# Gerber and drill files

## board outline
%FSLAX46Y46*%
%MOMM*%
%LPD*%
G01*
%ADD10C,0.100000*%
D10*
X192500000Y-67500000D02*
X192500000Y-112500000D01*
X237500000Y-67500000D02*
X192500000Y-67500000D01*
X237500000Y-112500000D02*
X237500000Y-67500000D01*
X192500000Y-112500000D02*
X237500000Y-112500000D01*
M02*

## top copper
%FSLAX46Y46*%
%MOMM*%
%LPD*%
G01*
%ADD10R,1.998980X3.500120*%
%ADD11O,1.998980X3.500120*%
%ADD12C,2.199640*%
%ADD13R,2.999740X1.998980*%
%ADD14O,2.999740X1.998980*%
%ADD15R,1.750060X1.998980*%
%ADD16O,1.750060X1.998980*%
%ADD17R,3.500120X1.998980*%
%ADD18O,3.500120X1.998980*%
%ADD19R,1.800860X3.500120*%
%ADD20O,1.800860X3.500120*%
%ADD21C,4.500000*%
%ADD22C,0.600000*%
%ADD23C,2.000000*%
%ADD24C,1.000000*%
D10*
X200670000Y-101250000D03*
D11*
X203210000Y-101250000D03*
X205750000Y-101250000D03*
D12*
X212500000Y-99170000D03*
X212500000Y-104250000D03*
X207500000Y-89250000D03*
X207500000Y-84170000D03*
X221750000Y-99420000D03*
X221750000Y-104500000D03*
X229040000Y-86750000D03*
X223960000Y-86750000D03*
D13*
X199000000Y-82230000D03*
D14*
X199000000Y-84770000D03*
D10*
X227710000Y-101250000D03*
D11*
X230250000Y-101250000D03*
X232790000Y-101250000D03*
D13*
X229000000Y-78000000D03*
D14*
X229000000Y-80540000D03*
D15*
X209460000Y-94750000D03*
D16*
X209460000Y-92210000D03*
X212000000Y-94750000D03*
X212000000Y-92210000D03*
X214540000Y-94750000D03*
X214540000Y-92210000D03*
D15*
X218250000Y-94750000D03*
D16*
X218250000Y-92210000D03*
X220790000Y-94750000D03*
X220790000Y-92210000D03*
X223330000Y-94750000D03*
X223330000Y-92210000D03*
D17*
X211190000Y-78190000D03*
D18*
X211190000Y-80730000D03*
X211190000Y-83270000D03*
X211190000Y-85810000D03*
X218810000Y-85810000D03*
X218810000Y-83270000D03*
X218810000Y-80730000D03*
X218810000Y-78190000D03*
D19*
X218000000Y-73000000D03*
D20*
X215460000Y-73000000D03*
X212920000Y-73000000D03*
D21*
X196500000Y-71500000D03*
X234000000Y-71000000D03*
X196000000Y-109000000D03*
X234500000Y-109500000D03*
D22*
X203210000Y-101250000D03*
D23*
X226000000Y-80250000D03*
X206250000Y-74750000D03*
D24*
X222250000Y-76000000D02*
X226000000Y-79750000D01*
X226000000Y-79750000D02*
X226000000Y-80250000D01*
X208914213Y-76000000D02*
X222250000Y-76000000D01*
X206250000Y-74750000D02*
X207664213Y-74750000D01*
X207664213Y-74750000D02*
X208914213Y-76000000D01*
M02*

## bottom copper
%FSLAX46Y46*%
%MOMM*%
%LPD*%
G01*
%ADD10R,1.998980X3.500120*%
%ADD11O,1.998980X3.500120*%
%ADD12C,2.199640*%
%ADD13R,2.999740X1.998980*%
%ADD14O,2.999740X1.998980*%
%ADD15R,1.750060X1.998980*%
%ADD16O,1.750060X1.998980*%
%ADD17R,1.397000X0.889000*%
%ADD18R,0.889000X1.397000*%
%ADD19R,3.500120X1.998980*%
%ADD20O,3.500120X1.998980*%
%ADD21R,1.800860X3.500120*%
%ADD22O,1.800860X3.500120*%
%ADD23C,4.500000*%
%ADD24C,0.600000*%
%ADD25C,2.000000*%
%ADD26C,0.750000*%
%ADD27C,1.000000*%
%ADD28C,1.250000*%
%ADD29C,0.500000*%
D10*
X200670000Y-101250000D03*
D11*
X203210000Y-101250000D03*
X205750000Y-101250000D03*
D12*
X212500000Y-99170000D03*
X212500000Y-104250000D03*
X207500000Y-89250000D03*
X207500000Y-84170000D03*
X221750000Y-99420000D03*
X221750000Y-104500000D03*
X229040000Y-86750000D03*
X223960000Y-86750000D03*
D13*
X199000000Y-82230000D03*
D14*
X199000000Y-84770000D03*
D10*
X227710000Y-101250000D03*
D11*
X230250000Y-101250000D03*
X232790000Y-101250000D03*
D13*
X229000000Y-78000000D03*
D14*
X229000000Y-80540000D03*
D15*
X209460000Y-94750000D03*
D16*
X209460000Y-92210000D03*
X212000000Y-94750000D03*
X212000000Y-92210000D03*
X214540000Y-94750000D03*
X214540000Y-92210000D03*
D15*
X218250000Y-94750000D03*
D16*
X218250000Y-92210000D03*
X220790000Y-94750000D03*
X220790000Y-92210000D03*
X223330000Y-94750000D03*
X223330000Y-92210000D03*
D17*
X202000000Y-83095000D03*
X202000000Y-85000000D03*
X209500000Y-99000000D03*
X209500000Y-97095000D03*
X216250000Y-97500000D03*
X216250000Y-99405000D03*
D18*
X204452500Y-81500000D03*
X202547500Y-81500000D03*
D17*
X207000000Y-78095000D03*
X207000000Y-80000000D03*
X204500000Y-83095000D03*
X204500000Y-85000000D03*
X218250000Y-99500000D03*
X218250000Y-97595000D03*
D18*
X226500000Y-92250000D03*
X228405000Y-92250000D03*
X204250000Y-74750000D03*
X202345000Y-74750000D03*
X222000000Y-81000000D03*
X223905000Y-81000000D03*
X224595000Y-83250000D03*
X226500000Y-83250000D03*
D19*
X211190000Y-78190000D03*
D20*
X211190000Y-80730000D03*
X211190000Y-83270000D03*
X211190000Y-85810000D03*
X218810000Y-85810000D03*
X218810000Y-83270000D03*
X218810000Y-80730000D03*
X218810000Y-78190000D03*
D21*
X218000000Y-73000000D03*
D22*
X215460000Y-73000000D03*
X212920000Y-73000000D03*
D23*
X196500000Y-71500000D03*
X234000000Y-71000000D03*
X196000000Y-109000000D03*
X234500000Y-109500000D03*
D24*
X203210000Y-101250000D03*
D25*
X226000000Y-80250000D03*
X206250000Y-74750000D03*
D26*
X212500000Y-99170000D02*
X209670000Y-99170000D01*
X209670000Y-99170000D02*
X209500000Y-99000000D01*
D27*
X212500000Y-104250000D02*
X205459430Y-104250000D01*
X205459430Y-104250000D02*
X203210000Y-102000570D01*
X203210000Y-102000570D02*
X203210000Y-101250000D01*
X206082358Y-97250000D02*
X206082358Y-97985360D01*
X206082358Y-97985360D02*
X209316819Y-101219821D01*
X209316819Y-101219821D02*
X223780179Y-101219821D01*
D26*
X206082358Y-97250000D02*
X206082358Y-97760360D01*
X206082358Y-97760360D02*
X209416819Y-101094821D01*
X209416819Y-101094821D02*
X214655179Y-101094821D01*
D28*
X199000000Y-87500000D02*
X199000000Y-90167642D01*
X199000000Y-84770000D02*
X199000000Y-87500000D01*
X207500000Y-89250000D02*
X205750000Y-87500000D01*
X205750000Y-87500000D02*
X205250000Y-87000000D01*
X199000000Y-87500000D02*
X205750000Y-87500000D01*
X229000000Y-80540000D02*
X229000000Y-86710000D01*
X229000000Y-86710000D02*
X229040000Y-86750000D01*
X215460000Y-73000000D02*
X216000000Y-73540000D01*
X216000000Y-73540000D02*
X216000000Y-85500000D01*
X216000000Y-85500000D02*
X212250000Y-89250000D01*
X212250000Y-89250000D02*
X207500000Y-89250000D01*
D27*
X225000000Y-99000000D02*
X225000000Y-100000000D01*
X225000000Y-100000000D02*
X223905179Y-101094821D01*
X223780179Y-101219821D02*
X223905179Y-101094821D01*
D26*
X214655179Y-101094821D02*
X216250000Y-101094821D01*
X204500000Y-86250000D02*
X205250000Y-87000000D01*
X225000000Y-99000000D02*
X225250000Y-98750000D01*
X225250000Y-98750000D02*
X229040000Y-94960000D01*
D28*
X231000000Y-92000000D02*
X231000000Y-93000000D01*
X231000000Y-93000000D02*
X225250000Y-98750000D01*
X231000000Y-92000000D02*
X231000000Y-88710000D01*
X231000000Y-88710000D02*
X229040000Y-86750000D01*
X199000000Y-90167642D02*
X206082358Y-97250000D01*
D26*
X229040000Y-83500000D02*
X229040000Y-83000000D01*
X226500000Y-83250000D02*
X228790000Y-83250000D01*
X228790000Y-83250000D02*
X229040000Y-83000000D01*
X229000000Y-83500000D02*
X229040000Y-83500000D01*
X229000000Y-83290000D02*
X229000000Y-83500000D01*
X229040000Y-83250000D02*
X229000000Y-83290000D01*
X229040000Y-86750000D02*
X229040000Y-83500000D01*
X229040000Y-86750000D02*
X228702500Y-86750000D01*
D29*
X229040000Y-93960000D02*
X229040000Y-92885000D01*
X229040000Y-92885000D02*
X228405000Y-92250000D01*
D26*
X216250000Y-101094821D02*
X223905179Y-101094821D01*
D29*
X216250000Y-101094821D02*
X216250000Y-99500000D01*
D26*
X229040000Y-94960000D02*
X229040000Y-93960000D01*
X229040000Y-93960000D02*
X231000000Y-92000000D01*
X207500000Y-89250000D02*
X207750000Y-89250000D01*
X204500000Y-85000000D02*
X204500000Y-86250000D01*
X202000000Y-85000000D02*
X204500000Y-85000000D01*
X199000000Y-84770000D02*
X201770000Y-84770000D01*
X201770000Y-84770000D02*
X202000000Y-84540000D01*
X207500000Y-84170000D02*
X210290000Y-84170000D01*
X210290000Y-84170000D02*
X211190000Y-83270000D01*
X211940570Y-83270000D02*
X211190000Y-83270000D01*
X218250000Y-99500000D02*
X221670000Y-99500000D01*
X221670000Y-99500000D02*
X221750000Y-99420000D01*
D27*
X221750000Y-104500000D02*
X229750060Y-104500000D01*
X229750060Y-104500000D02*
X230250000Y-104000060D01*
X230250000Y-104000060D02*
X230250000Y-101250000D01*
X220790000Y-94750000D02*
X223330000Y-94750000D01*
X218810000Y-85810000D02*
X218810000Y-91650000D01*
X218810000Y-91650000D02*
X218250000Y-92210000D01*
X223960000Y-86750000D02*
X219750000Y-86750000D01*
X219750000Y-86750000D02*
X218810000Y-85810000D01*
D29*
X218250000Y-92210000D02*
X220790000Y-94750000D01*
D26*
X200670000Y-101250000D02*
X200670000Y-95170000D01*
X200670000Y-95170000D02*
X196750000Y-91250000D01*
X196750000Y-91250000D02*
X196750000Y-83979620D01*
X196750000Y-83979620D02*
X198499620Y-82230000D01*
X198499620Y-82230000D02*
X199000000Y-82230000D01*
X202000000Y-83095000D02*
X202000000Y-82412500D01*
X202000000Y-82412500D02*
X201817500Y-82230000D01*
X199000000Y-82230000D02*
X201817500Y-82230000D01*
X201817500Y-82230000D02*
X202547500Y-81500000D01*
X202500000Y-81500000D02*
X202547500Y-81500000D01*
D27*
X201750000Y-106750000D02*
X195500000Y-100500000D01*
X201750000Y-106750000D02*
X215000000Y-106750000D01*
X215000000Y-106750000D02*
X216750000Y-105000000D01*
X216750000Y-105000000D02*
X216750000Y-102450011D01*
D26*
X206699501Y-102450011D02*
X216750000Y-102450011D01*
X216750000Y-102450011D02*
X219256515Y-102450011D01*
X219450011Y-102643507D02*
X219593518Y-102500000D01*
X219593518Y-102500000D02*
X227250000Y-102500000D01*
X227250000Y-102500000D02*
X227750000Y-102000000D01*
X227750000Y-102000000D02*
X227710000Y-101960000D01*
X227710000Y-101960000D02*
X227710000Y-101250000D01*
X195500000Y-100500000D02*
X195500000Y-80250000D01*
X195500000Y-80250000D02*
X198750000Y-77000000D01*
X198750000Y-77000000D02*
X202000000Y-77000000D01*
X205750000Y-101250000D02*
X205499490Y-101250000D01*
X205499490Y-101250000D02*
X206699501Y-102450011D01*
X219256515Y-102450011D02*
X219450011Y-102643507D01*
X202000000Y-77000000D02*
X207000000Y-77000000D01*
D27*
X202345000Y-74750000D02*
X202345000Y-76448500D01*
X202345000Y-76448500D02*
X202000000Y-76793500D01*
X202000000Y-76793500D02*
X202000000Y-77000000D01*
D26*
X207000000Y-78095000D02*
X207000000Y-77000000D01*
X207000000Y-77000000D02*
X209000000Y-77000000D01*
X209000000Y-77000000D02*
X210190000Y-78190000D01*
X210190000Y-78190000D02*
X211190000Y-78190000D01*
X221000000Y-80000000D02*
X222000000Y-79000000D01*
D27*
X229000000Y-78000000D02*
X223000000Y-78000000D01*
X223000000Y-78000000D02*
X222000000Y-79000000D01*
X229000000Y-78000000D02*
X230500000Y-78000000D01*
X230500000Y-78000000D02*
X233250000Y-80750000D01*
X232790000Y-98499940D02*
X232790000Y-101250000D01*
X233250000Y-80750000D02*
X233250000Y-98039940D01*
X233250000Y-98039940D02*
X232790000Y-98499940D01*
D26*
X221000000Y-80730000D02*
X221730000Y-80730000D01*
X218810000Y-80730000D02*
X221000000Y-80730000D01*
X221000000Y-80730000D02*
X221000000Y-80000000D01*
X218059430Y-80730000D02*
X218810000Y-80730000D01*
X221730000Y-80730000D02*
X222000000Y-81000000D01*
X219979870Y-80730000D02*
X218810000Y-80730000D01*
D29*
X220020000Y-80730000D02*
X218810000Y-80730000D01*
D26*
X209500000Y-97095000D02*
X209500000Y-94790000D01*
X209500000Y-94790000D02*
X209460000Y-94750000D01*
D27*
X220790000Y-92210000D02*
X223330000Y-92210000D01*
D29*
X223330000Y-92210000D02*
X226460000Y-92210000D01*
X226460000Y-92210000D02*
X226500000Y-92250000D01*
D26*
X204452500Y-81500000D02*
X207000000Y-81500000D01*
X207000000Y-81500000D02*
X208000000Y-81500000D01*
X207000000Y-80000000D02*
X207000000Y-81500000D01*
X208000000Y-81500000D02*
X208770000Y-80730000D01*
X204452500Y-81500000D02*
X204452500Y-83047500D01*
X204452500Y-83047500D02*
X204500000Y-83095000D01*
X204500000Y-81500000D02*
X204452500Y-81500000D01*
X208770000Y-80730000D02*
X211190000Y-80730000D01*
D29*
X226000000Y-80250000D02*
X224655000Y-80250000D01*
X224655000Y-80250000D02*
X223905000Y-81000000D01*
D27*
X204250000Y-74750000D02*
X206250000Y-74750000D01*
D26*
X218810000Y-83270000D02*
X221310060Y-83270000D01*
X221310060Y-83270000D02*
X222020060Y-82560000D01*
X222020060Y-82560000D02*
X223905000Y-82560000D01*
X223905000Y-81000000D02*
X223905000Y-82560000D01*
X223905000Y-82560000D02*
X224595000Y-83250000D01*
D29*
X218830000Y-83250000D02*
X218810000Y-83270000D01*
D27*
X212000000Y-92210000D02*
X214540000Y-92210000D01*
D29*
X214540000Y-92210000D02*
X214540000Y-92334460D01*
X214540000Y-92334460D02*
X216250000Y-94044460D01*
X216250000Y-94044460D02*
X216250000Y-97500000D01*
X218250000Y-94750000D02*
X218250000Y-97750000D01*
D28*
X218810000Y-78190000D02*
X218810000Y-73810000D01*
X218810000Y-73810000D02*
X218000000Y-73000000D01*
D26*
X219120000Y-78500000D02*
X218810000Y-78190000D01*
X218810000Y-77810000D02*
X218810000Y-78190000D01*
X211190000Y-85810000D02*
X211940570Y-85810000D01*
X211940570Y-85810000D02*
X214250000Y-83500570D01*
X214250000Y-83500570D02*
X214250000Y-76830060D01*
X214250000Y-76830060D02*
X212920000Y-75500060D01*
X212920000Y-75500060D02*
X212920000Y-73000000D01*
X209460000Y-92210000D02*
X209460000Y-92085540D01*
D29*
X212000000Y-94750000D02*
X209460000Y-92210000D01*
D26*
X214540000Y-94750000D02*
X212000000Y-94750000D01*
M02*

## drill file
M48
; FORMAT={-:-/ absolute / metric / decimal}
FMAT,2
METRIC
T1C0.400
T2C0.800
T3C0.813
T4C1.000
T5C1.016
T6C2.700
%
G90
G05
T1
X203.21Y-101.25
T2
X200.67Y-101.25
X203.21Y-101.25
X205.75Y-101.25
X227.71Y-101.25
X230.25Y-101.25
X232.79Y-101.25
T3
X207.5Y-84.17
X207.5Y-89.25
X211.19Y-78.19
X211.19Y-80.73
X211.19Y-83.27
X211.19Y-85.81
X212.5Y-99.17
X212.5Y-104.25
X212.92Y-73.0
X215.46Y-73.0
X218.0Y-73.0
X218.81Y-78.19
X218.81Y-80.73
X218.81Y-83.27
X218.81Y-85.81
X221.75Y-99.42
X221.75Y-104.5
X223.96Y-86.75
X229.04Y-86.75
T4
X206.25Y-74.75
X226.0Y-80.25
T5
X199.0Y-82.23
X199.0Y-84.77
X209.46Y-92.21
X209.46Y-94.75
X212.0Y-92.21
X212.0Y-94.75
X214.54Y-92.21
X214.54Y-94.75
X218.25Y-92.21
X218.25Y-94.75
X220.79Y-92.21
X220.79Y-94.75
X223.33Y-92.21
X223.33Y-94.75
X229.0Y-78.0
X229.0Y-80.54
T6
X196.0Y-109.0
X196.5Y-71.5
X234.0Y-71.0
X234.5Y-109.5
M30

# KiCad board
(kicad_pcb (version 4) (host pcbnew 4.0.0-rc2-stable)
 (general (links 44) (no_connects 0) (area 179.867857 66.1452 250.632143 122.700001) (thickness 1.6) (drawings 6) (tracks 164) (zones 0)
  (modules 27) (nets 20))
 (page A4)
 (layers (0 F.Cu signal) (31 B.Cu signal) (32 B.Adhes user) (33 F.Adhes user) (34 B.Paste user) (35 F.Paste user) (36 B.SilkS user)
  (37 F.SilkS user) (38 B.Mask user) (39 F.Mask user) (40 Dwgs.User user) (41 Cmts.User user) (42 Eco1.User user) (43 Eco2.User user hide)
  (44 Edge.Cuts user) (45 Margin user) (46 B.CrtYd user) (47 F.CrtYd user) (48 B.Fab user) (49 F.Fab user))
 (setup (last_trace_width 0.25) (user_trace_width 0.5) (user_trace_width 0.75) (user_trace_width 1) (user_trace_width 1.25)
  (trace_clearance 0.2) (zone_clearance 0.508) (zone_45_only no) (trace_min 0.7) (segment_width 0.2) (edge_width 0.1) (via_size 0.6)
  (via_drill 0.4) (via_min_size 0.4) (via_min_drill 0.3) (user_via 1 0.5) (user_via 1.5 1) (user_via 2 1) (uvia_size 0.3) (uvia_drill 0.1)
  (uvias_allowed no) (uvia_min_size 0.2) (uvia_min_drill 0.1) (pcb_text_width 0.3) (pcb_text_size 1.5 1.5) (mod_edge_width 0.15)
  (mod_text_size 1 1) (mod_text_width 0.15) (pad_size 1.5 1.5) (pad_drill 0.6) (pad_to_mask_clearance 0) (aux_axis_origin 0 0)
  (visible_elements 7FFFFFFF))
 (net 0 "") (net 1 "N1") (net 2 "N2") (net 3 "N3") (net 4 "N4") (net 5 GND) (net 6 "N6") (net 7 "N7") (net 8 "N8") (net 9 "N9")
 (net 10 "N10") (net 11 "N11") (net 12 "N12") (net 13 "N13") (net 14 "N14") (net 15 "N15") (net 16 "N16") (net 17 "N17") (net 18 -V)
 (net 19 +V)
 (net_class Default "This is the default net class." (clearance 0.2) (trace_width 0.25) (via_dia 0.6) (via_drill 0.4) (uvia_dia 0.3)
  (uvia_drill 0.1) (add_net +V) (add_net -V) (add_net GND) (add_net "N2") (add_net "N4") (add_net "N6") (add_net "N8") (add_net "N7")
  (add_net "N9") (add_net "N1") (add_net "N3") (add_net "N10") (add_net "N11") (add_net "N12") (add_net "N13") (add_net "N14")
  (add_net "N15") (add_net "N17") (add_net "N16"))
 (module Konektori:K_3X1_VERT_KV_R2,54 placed (layer F.Cu) (at 203.21 101.25)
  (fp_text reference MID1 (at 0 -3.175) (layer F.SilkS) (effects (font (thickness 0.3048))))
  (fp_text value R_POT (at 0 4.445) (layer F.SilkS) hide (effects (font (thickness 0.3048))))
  (pad 1 thru_hole rect (at -2.54 0) (size 1.99898 3.50012) (drill 0.8001) (layers *.Cu) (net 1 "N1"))
  (pad 2 thru_hole oval (at 0 0) (size 1.99898 3.50012) (drill 0.8001) (layers *.Cu) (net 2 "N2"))
  (pad 3 thru_hole oval (at 2.54 0) (size 1.99898 3.50012) (drill 0.8001) (layers *.Cu) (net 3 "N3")))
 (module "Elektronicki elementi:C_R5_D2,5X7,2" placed (layer F.Cu) (at 212.5 101.71 90)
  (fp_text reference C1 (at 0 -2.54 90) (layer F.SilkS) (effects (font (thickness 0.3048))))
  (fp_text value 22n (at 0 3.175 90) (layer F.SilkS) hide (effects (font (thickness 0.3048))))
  (pad 2 thru_hole circle (at 2.54 0 90) (size 2.19964 2.19964) (drill 0.8128) (layers *.Cu) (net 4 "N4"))
  (pad 1 thru_hole circle (at -2.54 0 90) (size 2.19964 2.19964) (drill 0.8128) (layers *.Cu) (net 2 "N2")))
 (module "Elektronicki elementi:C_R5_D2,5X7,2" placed (layer F.Cu) (at 207.5 86.71 270)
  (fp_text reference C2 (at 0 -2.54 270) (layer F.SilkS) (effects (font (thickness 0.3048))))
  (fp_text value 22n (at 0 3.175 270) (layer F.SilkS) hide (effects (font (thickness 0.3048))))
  (pad 2 thru_hole circle (at 2.54 0 270) (size 2.19964 2.19964) (drill 0.8128) (layers *.Cu) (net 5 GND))
  (pad 1 thru_hole circle (at -2.54 0 270) (size 2.19964 2.19964) (drill 0.8128) (layers *.Cu) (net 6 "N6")))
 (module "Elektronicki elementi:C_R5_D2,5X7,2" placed (layer F.Cu) (at 221.75 101.96 90)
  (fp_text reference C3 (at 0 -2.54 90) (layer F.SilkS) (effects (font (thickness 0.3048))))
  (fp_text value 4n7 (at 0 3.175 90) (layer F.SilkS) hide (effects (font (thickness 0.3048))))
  (pad 2 thru_hole circle (at 2.54 0 90) (size 2.19964 2.19964) (drill 0.8128) (layers *.Cu) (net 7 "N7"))
  (pad 1 thru_hole circle (at -2.54 0 90) (size 2.19964 2.19964) (drill 0.8128) (layers *.Cu) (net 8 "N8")))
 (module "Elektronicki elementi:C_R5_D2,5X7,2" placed (layer F.Cu) (at 226.5 86.75)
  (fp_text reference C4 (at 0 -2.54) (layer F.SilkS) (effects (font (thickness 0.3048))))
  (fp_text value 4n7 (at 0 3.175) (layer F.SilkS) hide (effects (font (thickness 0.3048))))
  (pad 2 thru_hole circle (at 2.54 0) (size 2.19964 2.19964) (drill 0.8128) (layers *.Cu) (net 5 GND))
  (pad 1 thru_hole circle (at -2.54 0) (size 2.19964 2.19964) (drill 0.8128) (layers *.Cu) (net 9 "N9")))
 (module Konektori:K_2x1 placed (layer F.Cu) (at 199 83.5 270)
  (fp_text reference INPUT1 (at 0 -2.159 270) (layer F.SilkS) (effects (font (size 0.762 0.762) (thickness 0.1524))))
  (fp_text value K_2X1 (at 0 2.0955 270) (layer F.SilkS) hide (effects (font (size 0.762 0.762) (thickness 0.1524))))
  (pad 1 thru_hole rect (at -1.27 0 270) (size 1.99898 2.99974) (drill 1.016) (layers *.Cu *.Mask) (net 1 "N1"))
  (pad 2 thru_hole oval (at 1.27 0 270) (size 1.99898 2.99974) (drill 1.016) (layers *.Cu *.Mask) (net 5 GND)))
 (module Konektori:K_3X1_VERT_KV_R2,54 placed (layer F.Cu) (at 230.25 101.25)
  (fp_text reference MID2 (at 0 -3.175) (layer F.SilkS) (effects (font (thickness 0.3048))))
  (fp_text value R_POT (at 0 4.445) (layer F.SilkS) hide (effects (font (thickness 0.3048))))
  (pad 1 thru_hole rect (at -2.54 0) (size 1.99898 3.50012) (drill 0.8001) (layers *.Cu) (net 3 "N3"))
  (pad 2 thru_hole oval (at 0 0) (size 1.99898 3.50012) (drill 0.8001) (layers *.Cu) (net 8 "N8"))
  (pad 3 thru_hole oval (at 2.54 0) (size 1.99898 3.50012) (drill 0.8001) (layers *.Cu) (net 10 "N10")))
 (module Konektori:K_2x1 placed (layer F.Cu) (at 229 79.27 270)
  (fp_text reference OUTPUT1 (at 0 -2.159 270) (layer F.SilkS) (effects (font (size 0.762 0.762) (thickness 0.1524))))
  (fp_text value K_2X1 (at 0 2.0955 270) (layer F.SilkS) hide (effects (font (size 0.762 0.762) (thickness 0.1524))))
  (pad 1 thru_hole rect (at -1.27 0 270) (size 1.99898 2.99974) (drill 1.016) (layers *.Cu *.Mask) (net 10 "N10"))
  (pad 2 thru_hole oval (at 1.27 0 270) (size 1.99898 2.99974) (drill 1.016) (layers *.Cu *.Mask) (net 5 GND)))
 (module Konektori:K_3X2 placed (layer F.Cu) (at 212 93.48)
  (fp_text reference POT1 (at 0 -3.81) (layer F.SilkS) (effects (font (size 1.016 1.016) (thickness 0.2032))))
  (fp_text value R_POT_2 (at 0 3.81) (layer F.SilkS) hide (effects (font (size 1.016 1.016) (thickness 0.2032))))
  (pad 1 thru_hole rect (at -2.54 1.27) (size 1.75006 1.99898) (drill 1.016) (layers *.Cu *.Mask F.SilkS) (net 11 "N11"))
  (pad 4 thru_hole oval (at -2.54 -1.27) (size 1.75006 1.99898) (drill 1.016) (layers *.Cu *.Mask F.SilkS) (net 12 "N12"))
  (pad 2 thru_hole oval (at 0 1.27) (size 1.75006 1.99898) (drill 1.016) (layers *.Cu *.Mask F.SilkS) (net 12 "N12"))
  (pad 5 thru_hole oval (at 0 -1.27) (size 1.75006 1.99898) (drill 1.016) (layers *.Cu *.Mask F.SilkS) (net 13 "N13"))
  (pad 3 thru_hole oval (at 2.54 1.27) (size 1.75006 1.99898) (drill 1.016) (layers *.Cu *.Mask F.SilkS) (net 12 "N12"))
  (pad 6 thru_hole oval (at 2.54 -1.27) (size 1.75006 1.99898) (drill 1.016) (layers *.Cu *.Mask F.SilkS) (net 13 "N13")))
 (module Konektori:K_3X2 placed (layer F.Cu) (at 220.79 93.48)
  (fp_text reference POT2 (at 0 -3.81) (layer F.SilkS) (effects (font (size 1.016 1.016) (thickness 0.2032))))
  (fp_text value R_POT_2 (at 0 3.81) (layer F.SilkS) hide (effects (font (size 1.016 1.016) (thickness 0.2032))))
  (pad 1 thru_hole rect (at -2.54 1.27) (size 1.75006 1.99898) (drill 1.016) (layers *.Cu *.Mask F.SilkS) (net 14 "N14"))
  (pad 4 thru_hole oval (at -2.54 -1.27) (size 1.75006 1.99898) (drill 1.016) (layers *.Cu *.Mask F.SilkS) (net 9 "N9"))
  (pad 2 thru_hole oval (at 0 1.27) (size 1.75006 1.99898) (drill 1.016) (layers *.Cu *.Mask F.SilkS) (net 9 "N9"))
  (pad 5 thru_hole oval (at 0 -1.27) (size 1.75006 1.99898) (drill 1.016) (layers *.Cu *.Mask F.SilkS) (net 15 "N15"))
  (pad 3 thru_hole oval (at 2.54 1.27) (size 1.75006 1.99898) (drill 1.016) (layers *.Cu *.Mask F.SilkS) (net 9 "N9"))
  (pad 6 thru_hole oval (at 2.54 -1.27) (size 1.75006 1.99898) (drill 1.016) (layers *.Cu *.Mask F.SilkS) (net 15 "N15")))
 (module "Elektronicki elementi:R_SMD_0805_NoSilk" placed (layer B.Cu) (at 202 84.0475 270)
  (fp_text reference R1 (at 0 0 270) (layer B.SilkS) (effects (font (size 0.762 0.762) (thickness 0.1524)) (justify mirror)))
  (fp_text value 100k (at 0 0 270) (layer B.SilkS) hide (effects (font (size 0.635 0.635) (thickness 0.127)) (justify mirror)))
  (pad 1 smd rect (at -0.9525 0 270) (size 0.889 1.397) (layers B.Cu B.Paste B.Mask) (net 1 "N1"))
  (pad 2 smd rect (at 0.9525 0 270) (size 0.889 1.397) (layers B.Cu B.Paste B.Mask) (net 5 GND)))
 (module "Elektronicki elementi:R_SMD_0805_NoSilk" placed (layer B.Cu) (at 209.5 98.0475 90)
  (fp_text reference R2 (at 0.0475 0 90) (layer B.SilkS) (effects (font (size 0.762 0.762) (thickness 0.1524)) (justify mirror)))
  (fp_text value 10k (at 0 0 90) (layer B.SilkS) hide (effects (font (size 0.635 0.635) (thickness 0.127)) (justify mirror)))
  (pad 1 smd rect (at -0.9525 0 90) (size 0.889 1.397) (layers B.Cu B.Paste B.Mask) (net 4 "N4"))
  (pad 2 smd rect (at 0.9525 0 90) (size 0.889 1.397) (layers B.Cu B.Paste B.Mask) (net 11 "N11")))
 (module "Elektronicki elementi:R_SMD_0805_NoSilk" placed (layer B.Cu) (at 216.25 98.4525 270)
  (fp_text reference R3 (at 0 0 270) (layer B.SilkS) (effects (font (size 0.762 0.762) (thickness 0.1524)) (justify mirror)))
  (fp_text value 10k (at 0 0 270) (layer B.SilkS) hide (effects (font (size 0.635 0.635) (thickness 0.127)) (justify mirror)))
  (pad 1 smd rect (at -0.9525 0 270) (size 0.889 1.397) (layers B.Cu B.Paste B.Mask) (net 13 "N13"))
  (pad 2 smd rect (at 0.9525 0 270) (size 0.889 1.397) (layers B.Cu B.Paste B.Mask) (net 5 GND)))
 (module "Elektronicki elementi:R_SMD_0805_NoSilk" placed (layer B.Cu) (at 203.5 81.5 180)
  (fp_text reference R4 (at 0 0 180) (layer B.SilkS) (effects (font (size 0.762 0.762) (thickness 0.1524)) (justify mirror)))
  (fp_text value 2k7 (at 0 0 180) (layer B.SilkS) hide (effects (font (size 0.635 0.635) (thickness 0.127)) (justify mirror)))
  (pad 1 smd rect (at -0.9525 0 180) (size 0.889 1.397) (layers B.Cu B.Paste B.Mask) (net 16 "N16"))
  (pad 2 smd rect (at 0.9525 0 180) (size 0.889 1.397) (layers B.Cu B.Paste B.Mask) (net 1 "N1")))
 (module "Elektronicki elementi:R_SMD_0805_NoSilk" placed (layer B.Cu) (at 207 79.0475 270)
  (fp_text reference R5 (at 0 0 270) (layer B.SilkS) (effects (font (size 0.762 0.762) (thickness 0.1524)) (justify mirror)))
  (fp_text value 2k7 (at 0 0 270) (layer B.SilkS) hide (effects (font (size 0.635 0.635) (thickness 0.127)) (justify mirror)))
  (pad 1 smd rect (at -0.9525 0 270) (size 0.889 1.397) (layers B.Cu B.Paste B.Mask) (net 3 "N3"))
  (pad 2 smd rect (at 0.9525 0 270) (size 0.889 1.397) (layers B.Cu B.Paste B.Mask) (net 16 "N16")))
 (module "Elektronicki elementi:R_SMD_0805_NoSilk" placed (layer B.Cu) (at 204.5 84.0475 270)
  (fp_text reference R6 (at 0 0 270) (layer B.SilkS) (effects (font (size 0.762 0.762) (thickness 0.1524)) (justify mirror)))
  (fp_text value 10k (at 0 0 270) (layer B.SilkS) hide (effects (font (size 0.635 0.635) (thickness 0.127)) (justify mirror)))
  (pad 1 smd rect (at -0.9525 0 270) (size 0.889 1.397) (layers B.Cu B.Paste B.Mask) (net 16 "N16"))
  (pad 2 smd rect (at 0.9525 0 270) (size 0.889 1.397) (layers B.Cu B.Paste B.Mask) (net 5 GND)))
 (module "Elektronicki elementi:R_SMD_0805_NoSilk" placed (layer B.Cu) (at 218.25 98.5475 90)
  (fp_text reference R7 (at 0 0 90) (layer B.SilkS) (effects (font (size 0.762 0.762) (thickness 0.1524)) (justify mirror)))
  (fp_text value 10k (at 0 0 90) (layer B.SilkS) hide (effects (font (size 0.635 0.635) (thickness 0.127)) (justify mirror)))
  (pad 1 smd rect (at -0.9525 0 90) (size 0.889 1.397) (layers B.Cu B.Paste B.Mask) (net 7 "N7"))
  (pad 2 smd rect (at 0.9525 0 90) (size 0.889 1.397) (layers B.Cu B.Paste B.Mask) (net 14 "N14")))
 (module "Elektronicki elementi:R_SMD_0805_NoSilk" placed (layer B.Cu) (at 227.4525 92.25)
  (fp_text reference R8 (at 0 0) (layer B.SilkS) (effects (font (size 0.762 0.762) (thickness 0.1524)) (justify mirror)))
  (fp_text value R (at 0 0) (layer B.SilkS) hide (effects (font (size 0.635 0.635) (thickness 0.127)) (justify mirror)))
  (pad 1 smd rect (at -0.9525 0) (size 0.889 1.397) (layers B.Cu B.Paste B.Mask) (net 15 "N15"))
  (pad 2 smd rect (at 0.9525 0) (size 0.889 1.397) (layers B.Cu B.Paste B.Mask) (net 5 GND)))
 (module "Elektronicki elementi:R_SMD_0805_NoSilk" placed (layer B.Cu) (at 203.2975 74.75 180)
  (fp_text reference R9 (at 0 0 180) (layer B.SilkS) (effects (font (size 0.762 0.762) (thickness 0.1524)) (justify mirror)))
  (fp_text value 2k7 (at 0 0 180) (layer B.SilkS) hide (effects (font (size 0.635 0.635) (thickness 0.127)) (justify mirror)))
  (pad 1 smd rect (at -0.9525 0 180) (size 0.889 1.397) (layers B.Cu B.Paste B.Mask) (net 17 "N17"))
  (pad 2 smd rect (at 0.9525 0 180) (size 0.889 1.397) (layers B.Cu B.Paste B.Mask) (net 3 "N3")))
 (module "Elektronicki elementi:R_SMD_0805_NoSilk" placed (layer B.Cu) (at 222.9525 81)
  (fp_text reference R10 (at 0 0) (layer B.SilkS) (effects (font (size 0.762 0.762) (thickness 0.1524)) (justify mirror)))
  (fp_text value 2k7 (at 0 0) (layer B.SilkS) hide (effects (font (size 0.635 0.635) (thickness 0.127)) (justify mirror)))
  (pad 1 smd rect (at -0.9525 0) (size 0.889 1.397) (layers B.Cu B.Paste B.Mask) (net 10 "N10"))
  (pad 2 smd rect (at 0.9525 0) (size 0.889 1.397) (layers B.Cu B.Paste B.Mask) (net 17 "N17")))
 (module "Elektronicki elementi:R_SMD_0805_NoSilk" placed (layer B.Cu) (at 225.5475 83.25)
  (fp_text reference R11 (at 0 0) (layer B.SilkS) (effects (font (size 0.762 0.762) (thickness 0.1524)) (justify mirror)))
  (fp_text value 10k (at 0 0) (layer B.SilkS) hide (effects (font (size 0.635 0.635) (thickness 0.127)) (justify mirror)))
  (pad 1 smd rect (at -0.9525 0) (size 0.889 1.397) (layers B.Cu B.Paste B.Mask) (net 17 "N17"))
  (pad 2 smd rect (at 0.9525 0) (size 0.889 1.397) (layers B.Cu B.Paste B.Mask) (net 5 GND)))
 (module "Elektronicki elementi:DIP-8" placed (layer F.Cu) (at 215 82 270)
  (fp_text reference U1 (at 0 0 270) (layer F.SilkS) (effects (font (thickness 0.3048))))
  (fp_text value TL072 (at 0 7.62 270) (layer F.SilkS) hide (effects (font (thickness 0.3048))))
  (pad 1 thru_hole rect (at -3.81 3.81 270) (size 1.99898 3.50012) (drill 0.8128) (layers *.Cu) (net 3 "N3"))
  (pad 2 thru_hole oval (at -1.27 3.81 270) (size 1.99898 3.50012) (drill 0.8128) (layers *.Cu) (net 16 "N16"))
  (pad 3 thru_hole oval (at 1.27 3.81 270) (size 1.99898 3.50012) (drill 0.8128) (layers *.Cu) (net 6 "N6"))
  (pad 4 thru_hole oval (at 3.81 3.81 270) (size 1.99898 3.50012) (drill 0.8128) (layers *.Cu) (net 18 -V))
  (pad 5 thru_hole oval (at 3.81 -3.81 270) (size 1.99898 3.50012) (drill 0.8128) (layers *.Cu) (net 9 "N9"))
  (pad 6 thru_hole oval (at 1.27 -3.81 270) (size 1.99898 3.50012) (drill 0.8128) (layers *.Cu) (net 17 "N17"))
  (pad 7 thru_hole oval (at -1.27 -3.81 270) (size 1.99898 3.50012) (drill 0.8128) (layers *.Cu) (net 10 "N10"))
  (pad 8 thru_hole oval (at -3.81 -3.81 270) (size 1.99898 3.50012) (drill 0.8128) (layers *.Cu) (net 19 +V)))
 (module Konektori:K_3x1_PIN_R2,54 (layer F.Cu) (at 215.46 73 180)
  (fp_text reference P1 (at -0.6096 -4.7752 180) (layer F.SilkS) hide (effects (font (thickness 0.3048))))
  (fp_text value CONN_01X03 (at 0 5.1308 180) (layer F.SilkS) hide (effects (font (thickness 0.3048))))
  (pad 1 thru_hole rect (at -2.54 0 180) (size 1.80086 3.50012) (drill 0.8128) (layers *.Cu *.Mask) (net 19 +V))
  (pad 2 thru_hole oval (at 0 0 180) (size 1.80086 3.50012) (drill 0.8128) (layers *.Cu *.Mask) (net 5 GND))
  (pad 3 thru_hole oval (at 2.54 0 180) (size 1.80086 3.50012) (drill 0.8128) (layers *.Cu *.Mask) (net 18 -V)))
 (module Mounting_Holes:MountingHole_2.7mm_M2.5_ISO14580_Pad (layer F.Cu) (at 196.5 71.5)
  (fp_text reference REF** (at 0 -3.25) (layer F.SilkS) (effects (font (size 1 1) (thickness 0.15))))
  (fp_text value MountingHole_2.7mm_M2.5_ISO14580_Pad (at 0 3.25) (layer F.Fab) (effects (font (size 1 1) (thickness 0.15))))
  (pad 1 thru_hole circle (at 0 0) (size 4.5 4.5) (drill 2.7) (layers *.Cu *.Mask F.SilkS)))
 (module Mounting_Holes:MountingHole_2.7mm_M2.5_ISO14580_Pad (layer F.Cu) (at 234 71)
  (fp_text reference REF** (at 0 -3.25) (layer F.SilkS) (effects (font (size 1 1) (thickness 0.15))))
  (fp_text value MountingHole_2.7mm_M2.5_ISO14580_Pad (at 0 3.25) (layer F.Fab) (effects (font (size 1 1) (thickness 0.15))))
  (pad 1 thru_hole circle (at 0 0) (size 4.5 4.5) (drill 2.7) (layers *.Cu *.Mask F.SilkS)))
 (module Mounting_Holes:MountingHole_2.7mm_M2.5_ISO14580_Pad (layer F.Cu) (at 196 109)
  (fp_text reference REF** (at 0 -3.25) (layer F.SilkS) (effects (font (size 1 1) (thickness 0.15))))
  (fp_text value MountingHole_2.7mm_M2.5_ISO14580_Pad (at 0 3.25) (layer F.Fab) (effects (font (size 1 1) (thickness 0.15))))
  (pad 1 thru_hole circle (at 0 0) (size 4.5 4.5) (drill 2.7) (layers *.Cu *.Mask F.SilkS)))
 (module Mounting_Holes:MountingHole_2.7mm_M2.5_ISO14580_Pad (layer F.Cu) (at 234.5 109.5)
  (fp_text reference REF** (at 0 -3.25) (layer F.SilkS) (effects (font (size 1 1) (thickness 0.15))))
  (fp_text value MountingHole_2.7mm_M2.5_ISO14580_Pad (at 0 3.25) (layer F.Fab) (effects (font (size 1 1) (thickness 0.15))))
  (pad 1 thru_hole circle (at 0 0) (size 4.5 4.5) (drill 2.7) (layers *.Cu *.Mask F.SilkS)))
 (gr_line (start 192.5 67.5) (end 192.5 112.5) (angle 90) (layer Edge.Cuts) (width 0.1))
 (gr_line (start 237.5 67.5) (end 192.5 67.5) (angle 90) (layer Edge.Cuts) (width 0.1))
 (gr_line (start 237.5 112.5) (end 237.5 67.5) (angle 90) (layer Edge.Cuts) (width 0.1))
 (gr_line (start 192.5 112.5) (end 237.5 112.5) (angle 90) (layer Edge.Cuts) (width 0.1))
 (segment (start 212.5 99.17) (end 209.67 99.17) (width 0.75) (layer B.Cu) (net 4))
 (segment (start 209.67 99.17) (end 209.5 99) (width 0.75) (layer B.Cu) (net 4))
 (segment (start 212.5 104.25) (end 205.45943 104.25) (width 1) (layer B.Cu) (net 2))
 (segment (start 205.45943 104.25) (end 203.21 102.00057) (width 1) (layer B.Cu) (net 2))
 (segment (start 203.21 102.00057) (end 203.21 101.25) (width 1) (layer B.Cu) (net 2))
 (via (at 203.21 101.25) (size 0.6) (drill 0.4) (layers F.Cu B.Cu) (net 2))
 (segment (start 206.082358 97.25) (end 206.082358 97.98536) (width 1) (layer B.Cu) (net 5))
 (segment (start 206.082358 97.98536) (end 209.316819 101.219821) (width 1) (layer B.Cu) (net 5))
 (segment (start 209.316819 101.219821) (end 223.780179 101.219821) (width 1) (layer B.Cu) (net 5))
 (segment (start 206.082358 97.25) (end 206.082358 97.76036) (width 0.75) (layer B.Cu) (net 5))
 (segment (start 206.082358 97.76036) (end 209.416819 101.094821) (width 0.75) (layer B.Cu) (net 5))
 (segment (start 209.416819 101.094821) (end 214.655179 101.094821) (width 0.75) (layer B.Cu) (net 5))
 (segment (start 199 87.5) (end 199 90.167642) (width 1.25) (layer B.Cu) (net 5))
 (segment (start 199 84.77) (end 199 87.5) (width 1.25) (layer B.Cu) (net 5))
 (segment (start 207.5 89.25) (end 205.75 87.5) (width 1.25) (layer B.Cu) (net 5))
 (segment (start 205.75 87.5) (end 205.25 87) (width 1.25) (layer B.Cu) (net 5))
 (segment (start 199 87.5) (end 205.75 87.5) (width 1.25) (layer B.Cu) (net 5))
 (segment (start 229 80.54) (end 229 86.71) (width 1.25) (layer B.Cu) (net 5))
 (segment (start 229 86.71) (end 229.04 86.75) (width 1.25) (layer B.Cu) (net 5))
 (segment (start 215.46 73) (end 216 73.54) (width 1.25) (layer B.Cu) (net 5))
 (segment (start 216 73.54) (end 216 85.5) (width 1.25) (layer B.Cu) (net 5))
 (segment (start 216 85.5) (end 212.25 89.25) (width 1.25) (layer B.Cu) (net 5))
 (segment (start 212.25 89.25) (end 207.5 89.25) (width 1.25) (layer B.Cu) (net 5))
 (segment (start 225 99) (end 225 100) (width 1) (layer B.Cu) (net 5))
 (segment (start 225 100) (end 223.905179 101.094821) (width 1) (layer B.Cu) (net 5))
 (segment (start 223.780179 101.219821) (end 223.905179 101.094821) (width 1) (layer B.Cu) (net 5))
 (segment (start 214.655179 101.094821) (end 216.25 101.094821) (width 0.75) (layer B.Cu) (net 5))
 (segment (start 204.5 86.25) (end 205.25 87) (width 0.75) (layer B.Cu) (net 5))
 (segment (start 225 99) (end 225.25 98.75) (width 0.75) (layer B.Cu) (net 5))
 (segment (start 225.25 98.75) (end 229.04 94.96) (width 0.75) (layer B.Cu) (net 5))
 (segment (start 231 92) (end 231 93) (width 1.25) (layer B.Cu) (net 5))
 (segment (start 231 93) (end 225.25 98.75) (width 1.25) (layer B.Cu) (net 5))
 (segment (start 231 92) (end 231 88.71) (width 1.25) (layer B.Cu) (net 5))
 (segment (start 231 88.71) (end 229.04 86.75) (width 1.25) (layer B.Cu) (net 5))
 (segment (start 199 90.167642) (end 206.082358 97.25) (width 1.25) (layer B.Cu) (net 5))
 (segment (start 229.04 83.5) (end 229.04 83) (width 0.75) (layer B.Cu) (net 5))
 (segment (start 226.5 83.25) (end 228.79 83.25) (width 0.75) (layer B.Cu) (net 5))
 (segment (start 228.79 83.25) (end 229.04 83) (width 0.75) (layer B.Cu) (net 5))
 (segment (start 229 83.5) (end 229.04 83.5) (width 0.75) (layer B.Cu) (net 5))
 (segment (start 229 83.29) (end 229 83.5) (width 0.75) (layer B.Cu) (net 5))
 (segment (start 229.04 83.25) (end 229 83.29) (width 0.75) (layer B.Cu) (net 5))
 (segment (start 229.04 86.75) (end 229.04 83.5) (width 0.75) (layer B.Cu) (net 5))
 (segment (start 229.04 86.75) (end 228.7025 86.75) (width 0.75) (layer B.Cu) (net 5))
 (segment (start 229.04 93.96) (end 229.04 92.885) (width 0.5) (layer B.Cu) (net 5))
 (segment (start 229.04 92.885) (end 228.405 92.25) (width 0.5) (layer B.Cu) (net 5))
 (segment (start 216.25 101.094821) (end 223.905179 101.094821) (width 0.75) (layer B.Cu) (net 5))
 (segment (start 216.25 101.094821) (end 216.25 99.5) (width 0.5) (layer B.Cu) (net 5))
 (segment (start 229.04 94.96) (end 229.04 93.96) (width 0.75) (layer B.Cu) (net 5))
 (segment (start 229.04 93.96) (end 231 92) (width 0.75) (layer B.Cu) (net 5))
 (segment (start 207.5 89.25) (end 207.75 89.25) (width 0.75) (layer B.Cu) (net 5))
 (segment (start 204.5 85) (end 204.5 86.25) (width 0.75) (layer B.Cu) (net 5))
 (segment (start 202 85) (end 204.5 85) (width 0.75) (layer B.Cu) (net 5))
 (segment (start 199 84.77) (end 201.77 84.77) (width 0.75) (layer B.Cu) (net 5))
 (segment (start 201.77 84.77) (end 202 84.54) (width 0.75) (layer B.Cu) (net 5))
 (segment (start 207.5 84.17) (end 210.29 84.17) (width 0.75) (layer B.Cu) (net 6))
 (segment (start 210.29 84.17) (end 211.19 83.27) (width 0.75) (layer B.Cu) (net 6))
 (segment (start 211.94057 83.27) (end 211.19 83.27) (width 0.75) (layer B.Cu) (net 6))
 (segment (start 218.25 99.5) (end 221.67 99.5) (width 0.75) (layer B.Cu) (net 7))
 (segment (start 221.67 99.5) (end 221.75 99.42) (width 0.75) (layer B.Cu) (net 7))
 (segment (start 221.75 104.5) (end 229.75006 104.5) (width 1) (layer B.Cu) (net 8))
 (segment (start 229.75006 104.5) (end 230.25 104.00006) (width 1) (layer B.Cu) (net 8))
 (segment (start 230.25 104.00006) (end 230.25 101.25) (width 1) (layer B.Cu) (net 8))
 (segment (start 220.79 94.75) (end 223.33 94.75) (width 1) (layer B.Cu) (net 9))
 (segment (start 218.81 85.81) (end 218.81 91.65) (width 1) (layer B.Cu) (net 9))
 (segment (start 218.81 91.65) (end 218.25 92.21) (width 1) (layer B.Cu) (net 9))
 (segment (start 223.96 86.75) (end 219.75 86.75) (width 1) (layer B.Cu) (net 9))
 (segment (start 219.75 86.75) (end 218.81 85.81) (width 1) (layer B.Cu) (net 9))
 (segment (start 218.25 92.21) (end 220.79 94.75) (width 0.5) (layer B.Cu) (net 9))
 (segment (start 200.67 101.25) (end 200.67 95.17) (width 0.75) (layer B.Cu) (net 1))
 (segment (start 200.67 95.17) (end 196.75 91.25) (width 0.75) (layer B.Cu) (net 1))
 (segment (start 196.75 91.25) (end 196.75 83.97962) (width 0.75) (layer B.Cu) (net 1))
 (segment (start 196.75 83.97962) (end 198.49962 82.23) (width 0.75) (layer B.Cu) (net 1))
 (segment (start 198.49962 82.23) (end 199 82.23) (width 0.75) (layer B.Cu) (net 1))
 (segment (start 202 83.095) (end 202 82.4125) (width 0.75) (layer B.Cu) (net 1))
 (segment (start 202 82.4125) (end 201.8175 82.23) (width 0.75) (layer B.Cu) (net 1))
 (segment (start 199 82.23) (end 201.8175 82.23) (width 0.75) (layer B.Cu) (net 1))
 (segment (start 201.8175 82.23) (end 202.5475 81.5) (width 0.75) (layer B.Cu) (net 1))
 (segment (start 202.5 81.5) (end 202.5475 81.5) (width 0.75) (layer B.Cu) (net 1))
 (segment (start 201.75 106.75) (end 195.5 100.5) (width 1) (layer B.Cu) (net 3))
 (segment (start 201.75 106.75) (end 215 106.75) (width 1) (layer B.Cu) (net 3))
 (segment (start 215 106.75) (end 216.75 105) (width 1) (layer B.Cu) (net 3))
 (segment (start 216.75 105) (end 216.75 102.450011) (width 1) (layer B.Cu) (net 3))
 (segment (start 206.699501 102.450011) (end 216.75 102.450011) (width 0.75) (layer B.Cu) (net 3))
 (segment (start 216.75 102.450011) (end 219.256515 102.450011) (width 0.75) (layer B.Cu) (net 3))
 (segment (start 219.450011 102.643507) (end 219.593518 102.5) (width 0.75) (layer B.Cu) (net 3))
 (segment (start 219.593518 102.5) (end 227.25 102.5) (width 0.75) (layer B.Cu) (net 3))
 (segment (start 227.25 102.5) (end 227.75 102) (width 0.75) (layer B.Cu) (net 3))
 (segment (start 227.75 102) (end 227.71 101.96) (width 0.75) (layer B.Cu) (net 3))
 (segment (start 227.71 101.96) (end 227.71 101.25) (width 0.75) (layer B.Cu) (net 3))
 (segment (start 195.5 100.5) (end 195.5 80.25) (width 0.75) (layer B.Cu) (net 3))
 (segment (start 195.5 80.25) (end 198.75 77) (width 0.75) (layer B.Cu) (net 3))
 (segment (start 198.75 77) (end 202 77) (width 0.75) (layer B.Cu) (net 3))
 (segment (start 205.75 101.25) (end 205.49949 101.25) (width 0.75) (layer B.Cu) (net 3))
 (segment (start 205.49949 101.25) (end 206.699501 102.450011) (width 0.75) (layer B.Cu) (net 3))
 (segment (start 219.256515 102.450011) (end 219.450011 102.643507) (width 0.75) (layer B.Cu) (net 3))
 (segment (start 202 77) (end 207 77) (width 0.75) (layer B.Cu) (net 3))
 (segment (start 202.345 74.75) (end 202.345 76.4485) (width 1) (layer B.Cu) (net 3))
 (segment (start 202.345 76.4485) (end 202 76.7935) (width 1) (layer B.Cu) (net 3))
 (segment (start 202 76.7935) (end 202 77) (width 1) (layer B.Cu) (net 3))
 (segment (start 207 78.095) (end 207 77) (width 0.75) (layer B.Cu) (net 3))
 (segment (start 207 77) (end 209 77) (width 0.75) (layer B.Cu) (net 3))
 (segment (start 209 77) (end 210.19 78.19) (width 0.75) (layer B.Cu) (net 3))
 (segment (start 210.19 78.19) (end 211.19 78.19) (width 0.75) (layer B.Cu) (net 3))
 (segment (start 221 80) (end 222 79) (width 0.75) (layer B.Cu) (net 10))
 (segment (start 229 78) (end 223 78) (width 1) (layer B.Cu) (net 10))
 (segment (start 223 78) (end 222 79) (width 1) (layer B.Cu) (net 10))
 (segment (start 229 78) (end 230.5 78) (width 1) (layer B.Cu) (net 10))
 (segment (start 230.5 78) (end 233.25 80.75) (width 1) (layer B.Cu) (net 10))
 (segment (start 232.79 98.49994) (end 232.79 101.25) (width 1) (layer B.Cu) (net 10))
 (segment (start 233.25 80.75) (end 233.25 98.03994) (width 1) (layer B.Cu) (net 10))
 (segment (start 233.25 98.03994) (end 232.79 98.49994) (width 1) (layer B.Cu) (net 10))
 (segment (start 221 80.73) (end 221.73 80.73) (width 0.75) (layer B.Cu) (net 10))
 (segment (start 218.81 80.73) (end 221 80.73) (width 0.75) (layer B.Cu) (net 10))
 (segment (start 221 80.73) (end 221 80) (width 0.75) (layer B.Cu) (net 10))
 (segment (start 218.05943 80.73) (end 218.81 80.73) (width 0.75) (layer B.Cu) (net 10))
 (segment (start 221.73 80.73) (end 222 81) (width 0.75) (layer B.Cu) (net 10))
 (segment (start 219.97987 80.73) (end 218.81 80.73) (width 0.75) (layer B.Cu) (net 10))
 (segment (start 220.02 80.73) (end 218.81 80.73) (width 0.5) (layer B.Cu) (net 10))
 (segment (start 209.5 97.095) (end 209.5 94.79) (width 0.75) (layer B.Cu) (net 11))
 (segment (start 209.5 94.79) (end 209.46 94.75) (width 0.75) (layer B.Cu) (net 11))
 (segment (start 220.79 92.21) (end 223.33 92.21) (width 1) (layer B.Cu) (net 15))
 (segment (start 223.33 92.21) (end 226.46 92.21) (width 0.5) (layer B.Cu) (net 15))
 (segment (start 226.46 92.21) (end 226.5 92.25) (width 0.5) (layer B.Cu) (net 15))
 (segment (start 204.4525 81.5) (end 207 81.5) (width 0.75) (layer B.Cu) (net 16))
 (segment (start 207 81.5) (end 208 81.5) (width 0.75) (layer B.Cu) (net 16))
 (segment (start 207 80) (end 207 81.5) (width 0.75) (layer B.Cu) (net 16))
 (segment (start 208 81.5) (end 208.77 80.73) (width 0.75) (layer B.Cu) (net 16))
 (segment (start 204.4525 81.5) (end 204.4525 83.0475) (width 0.75) (layer B.Cu) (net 16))
 (segment (start 204.4525 83.0475) (end 204.5 83.095) (width 0.75) (layer B.Cu) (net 16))
 (segment (start 204.5 81.5) (end 204.4525 81.5) (width 0.75) (layer B.Cu) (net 16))
 (segment (start 208.77 80.73) (end 211.19 80.73) (width 0.75) (layer B.Cu) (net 16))
 (segment (start 226 80.25) (end 224.655 80.25) (width 0.5) (layer B.Cu) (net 17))
 (segment (start 224.655 80.25) (end 223.905 81) (width 0.5) (layer B.Cu) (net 17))
 (segment (start 222.25 76) (end 226 79.75) (width 1) (layer F.Cu) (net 17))
 (segment (start 226 79.75) (end 226 80.25) (width 1) (layer F.Cu) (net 17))
 (via (at 226 80.25) (size 2) (drill 1) (layers F.Cu B.Cu) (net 17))
 (segment (start 208.914213 76) (end 222.25 76) (width 1) (layer F.Cu) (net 17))
 (segment (start 206.25 74.75) (end 207.664213 74.75) (width 1) (layer F.Cu) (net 17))
 (segment (start 207.664213 74.75) (end 208.914213 76) (width 1) (layer F.Cu) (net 17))
 (via (at 206.25 74.75) (size 2) (drill 1) (layers F.Cu B.Cu) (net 17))
 (segment (start 204.25 74.75) (end 206.25 74.75) (width 1) (layer B.Cu) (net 17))
 (segment (start 218.81 83.27) (end 221.31006 83.27) (width 0.75) (layer B.Cu) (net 17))
 (segment (start 221.31006 83.27) (end 222.02006 82.56) (width 0.75) (layer B.Cu) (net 17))
 (segment (start 222.02006 82.56) (end 223.905 82.56) (width 0.75) (layer B.Cu) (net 17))
 (segment (start 223.905 81) (end 223.905 82.56) (width 0.75) (layer B.Cu) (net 17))
 (segment (start 223.905 82.56) (end 224.595 83.25) (width 0.75) (layer B.Cu) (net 17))
 (segment (start 218.83 83.25) (end 218.81 83.27) (width 0.5) (layer B.Cu) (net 17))
 (segment (start 212 92.21) (end 214.54 92.21) (width 1) (layer B.Cu) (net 13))
 (segment (start 214.54 92.21) (end 214.54 92.33446) (width 0.5) (layer B.Cu) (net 13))
 (segment (start 214.54 92.33446) (end 216.25 94.04446) (width 0.5) (layer B.Cu) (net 13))
 (segment (start 216.25 94.04446) (end 216.25 97.5) (width 0.5) (layer B.Cu) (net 13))
 (segment (start 218.25 94.75) (end 218.25 97.75) (width 0.5) (layer B.Cu) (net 14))
 (segment (start 218.81 78.19) (end 218.81 73.81) (width 1.25) (layer B.Cu) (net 19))
 (segment (start 218.81 73.81) (end 218 73) (width 1.25) (layer B.Cu) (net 19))
 (segment (start 219.12 78.5) (end 218.81 78.19) (width 0.75) (layer B.Cu) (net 19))
 (segment (start 218.81 77.81) (end 218.81 78.19) (width 0.75) (layer B.Cu) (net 19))
 (segment (start 211.19 85.81) (end 211.94057 85.81) (width 0.75) (layer B.Cu) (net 18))
 (segment (start 211.94057 85.81) (end 214.25 83.50057) (width 0.75) (layer B.Cu) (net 18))
 (segment (start 214.25 83.50057) (end 214.25 76.83006) (width 0.75) (layer B.Cu) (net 18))
 (segment (start 214.25 76.83006) (end 212.92 75.50006) (width 0.75) (layer B.Cu) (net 18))
 (segment (start 212.92 75.50006) (end 212.92 73) (width 0.75) (layer B.Cu) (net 18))
 (segment (start 209.46 92.21) (end 209.46 92.08554) (width 0.75) (layer B.Cu) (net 12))
 (segment (start 212 94.75) (end 209.46 92.21) (width 0.5) (layer B.Cu) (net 12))
 (segment (start 214.54 94.75) (end 212 94.75) (width 0.75) (layer B.Cu) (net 12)))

